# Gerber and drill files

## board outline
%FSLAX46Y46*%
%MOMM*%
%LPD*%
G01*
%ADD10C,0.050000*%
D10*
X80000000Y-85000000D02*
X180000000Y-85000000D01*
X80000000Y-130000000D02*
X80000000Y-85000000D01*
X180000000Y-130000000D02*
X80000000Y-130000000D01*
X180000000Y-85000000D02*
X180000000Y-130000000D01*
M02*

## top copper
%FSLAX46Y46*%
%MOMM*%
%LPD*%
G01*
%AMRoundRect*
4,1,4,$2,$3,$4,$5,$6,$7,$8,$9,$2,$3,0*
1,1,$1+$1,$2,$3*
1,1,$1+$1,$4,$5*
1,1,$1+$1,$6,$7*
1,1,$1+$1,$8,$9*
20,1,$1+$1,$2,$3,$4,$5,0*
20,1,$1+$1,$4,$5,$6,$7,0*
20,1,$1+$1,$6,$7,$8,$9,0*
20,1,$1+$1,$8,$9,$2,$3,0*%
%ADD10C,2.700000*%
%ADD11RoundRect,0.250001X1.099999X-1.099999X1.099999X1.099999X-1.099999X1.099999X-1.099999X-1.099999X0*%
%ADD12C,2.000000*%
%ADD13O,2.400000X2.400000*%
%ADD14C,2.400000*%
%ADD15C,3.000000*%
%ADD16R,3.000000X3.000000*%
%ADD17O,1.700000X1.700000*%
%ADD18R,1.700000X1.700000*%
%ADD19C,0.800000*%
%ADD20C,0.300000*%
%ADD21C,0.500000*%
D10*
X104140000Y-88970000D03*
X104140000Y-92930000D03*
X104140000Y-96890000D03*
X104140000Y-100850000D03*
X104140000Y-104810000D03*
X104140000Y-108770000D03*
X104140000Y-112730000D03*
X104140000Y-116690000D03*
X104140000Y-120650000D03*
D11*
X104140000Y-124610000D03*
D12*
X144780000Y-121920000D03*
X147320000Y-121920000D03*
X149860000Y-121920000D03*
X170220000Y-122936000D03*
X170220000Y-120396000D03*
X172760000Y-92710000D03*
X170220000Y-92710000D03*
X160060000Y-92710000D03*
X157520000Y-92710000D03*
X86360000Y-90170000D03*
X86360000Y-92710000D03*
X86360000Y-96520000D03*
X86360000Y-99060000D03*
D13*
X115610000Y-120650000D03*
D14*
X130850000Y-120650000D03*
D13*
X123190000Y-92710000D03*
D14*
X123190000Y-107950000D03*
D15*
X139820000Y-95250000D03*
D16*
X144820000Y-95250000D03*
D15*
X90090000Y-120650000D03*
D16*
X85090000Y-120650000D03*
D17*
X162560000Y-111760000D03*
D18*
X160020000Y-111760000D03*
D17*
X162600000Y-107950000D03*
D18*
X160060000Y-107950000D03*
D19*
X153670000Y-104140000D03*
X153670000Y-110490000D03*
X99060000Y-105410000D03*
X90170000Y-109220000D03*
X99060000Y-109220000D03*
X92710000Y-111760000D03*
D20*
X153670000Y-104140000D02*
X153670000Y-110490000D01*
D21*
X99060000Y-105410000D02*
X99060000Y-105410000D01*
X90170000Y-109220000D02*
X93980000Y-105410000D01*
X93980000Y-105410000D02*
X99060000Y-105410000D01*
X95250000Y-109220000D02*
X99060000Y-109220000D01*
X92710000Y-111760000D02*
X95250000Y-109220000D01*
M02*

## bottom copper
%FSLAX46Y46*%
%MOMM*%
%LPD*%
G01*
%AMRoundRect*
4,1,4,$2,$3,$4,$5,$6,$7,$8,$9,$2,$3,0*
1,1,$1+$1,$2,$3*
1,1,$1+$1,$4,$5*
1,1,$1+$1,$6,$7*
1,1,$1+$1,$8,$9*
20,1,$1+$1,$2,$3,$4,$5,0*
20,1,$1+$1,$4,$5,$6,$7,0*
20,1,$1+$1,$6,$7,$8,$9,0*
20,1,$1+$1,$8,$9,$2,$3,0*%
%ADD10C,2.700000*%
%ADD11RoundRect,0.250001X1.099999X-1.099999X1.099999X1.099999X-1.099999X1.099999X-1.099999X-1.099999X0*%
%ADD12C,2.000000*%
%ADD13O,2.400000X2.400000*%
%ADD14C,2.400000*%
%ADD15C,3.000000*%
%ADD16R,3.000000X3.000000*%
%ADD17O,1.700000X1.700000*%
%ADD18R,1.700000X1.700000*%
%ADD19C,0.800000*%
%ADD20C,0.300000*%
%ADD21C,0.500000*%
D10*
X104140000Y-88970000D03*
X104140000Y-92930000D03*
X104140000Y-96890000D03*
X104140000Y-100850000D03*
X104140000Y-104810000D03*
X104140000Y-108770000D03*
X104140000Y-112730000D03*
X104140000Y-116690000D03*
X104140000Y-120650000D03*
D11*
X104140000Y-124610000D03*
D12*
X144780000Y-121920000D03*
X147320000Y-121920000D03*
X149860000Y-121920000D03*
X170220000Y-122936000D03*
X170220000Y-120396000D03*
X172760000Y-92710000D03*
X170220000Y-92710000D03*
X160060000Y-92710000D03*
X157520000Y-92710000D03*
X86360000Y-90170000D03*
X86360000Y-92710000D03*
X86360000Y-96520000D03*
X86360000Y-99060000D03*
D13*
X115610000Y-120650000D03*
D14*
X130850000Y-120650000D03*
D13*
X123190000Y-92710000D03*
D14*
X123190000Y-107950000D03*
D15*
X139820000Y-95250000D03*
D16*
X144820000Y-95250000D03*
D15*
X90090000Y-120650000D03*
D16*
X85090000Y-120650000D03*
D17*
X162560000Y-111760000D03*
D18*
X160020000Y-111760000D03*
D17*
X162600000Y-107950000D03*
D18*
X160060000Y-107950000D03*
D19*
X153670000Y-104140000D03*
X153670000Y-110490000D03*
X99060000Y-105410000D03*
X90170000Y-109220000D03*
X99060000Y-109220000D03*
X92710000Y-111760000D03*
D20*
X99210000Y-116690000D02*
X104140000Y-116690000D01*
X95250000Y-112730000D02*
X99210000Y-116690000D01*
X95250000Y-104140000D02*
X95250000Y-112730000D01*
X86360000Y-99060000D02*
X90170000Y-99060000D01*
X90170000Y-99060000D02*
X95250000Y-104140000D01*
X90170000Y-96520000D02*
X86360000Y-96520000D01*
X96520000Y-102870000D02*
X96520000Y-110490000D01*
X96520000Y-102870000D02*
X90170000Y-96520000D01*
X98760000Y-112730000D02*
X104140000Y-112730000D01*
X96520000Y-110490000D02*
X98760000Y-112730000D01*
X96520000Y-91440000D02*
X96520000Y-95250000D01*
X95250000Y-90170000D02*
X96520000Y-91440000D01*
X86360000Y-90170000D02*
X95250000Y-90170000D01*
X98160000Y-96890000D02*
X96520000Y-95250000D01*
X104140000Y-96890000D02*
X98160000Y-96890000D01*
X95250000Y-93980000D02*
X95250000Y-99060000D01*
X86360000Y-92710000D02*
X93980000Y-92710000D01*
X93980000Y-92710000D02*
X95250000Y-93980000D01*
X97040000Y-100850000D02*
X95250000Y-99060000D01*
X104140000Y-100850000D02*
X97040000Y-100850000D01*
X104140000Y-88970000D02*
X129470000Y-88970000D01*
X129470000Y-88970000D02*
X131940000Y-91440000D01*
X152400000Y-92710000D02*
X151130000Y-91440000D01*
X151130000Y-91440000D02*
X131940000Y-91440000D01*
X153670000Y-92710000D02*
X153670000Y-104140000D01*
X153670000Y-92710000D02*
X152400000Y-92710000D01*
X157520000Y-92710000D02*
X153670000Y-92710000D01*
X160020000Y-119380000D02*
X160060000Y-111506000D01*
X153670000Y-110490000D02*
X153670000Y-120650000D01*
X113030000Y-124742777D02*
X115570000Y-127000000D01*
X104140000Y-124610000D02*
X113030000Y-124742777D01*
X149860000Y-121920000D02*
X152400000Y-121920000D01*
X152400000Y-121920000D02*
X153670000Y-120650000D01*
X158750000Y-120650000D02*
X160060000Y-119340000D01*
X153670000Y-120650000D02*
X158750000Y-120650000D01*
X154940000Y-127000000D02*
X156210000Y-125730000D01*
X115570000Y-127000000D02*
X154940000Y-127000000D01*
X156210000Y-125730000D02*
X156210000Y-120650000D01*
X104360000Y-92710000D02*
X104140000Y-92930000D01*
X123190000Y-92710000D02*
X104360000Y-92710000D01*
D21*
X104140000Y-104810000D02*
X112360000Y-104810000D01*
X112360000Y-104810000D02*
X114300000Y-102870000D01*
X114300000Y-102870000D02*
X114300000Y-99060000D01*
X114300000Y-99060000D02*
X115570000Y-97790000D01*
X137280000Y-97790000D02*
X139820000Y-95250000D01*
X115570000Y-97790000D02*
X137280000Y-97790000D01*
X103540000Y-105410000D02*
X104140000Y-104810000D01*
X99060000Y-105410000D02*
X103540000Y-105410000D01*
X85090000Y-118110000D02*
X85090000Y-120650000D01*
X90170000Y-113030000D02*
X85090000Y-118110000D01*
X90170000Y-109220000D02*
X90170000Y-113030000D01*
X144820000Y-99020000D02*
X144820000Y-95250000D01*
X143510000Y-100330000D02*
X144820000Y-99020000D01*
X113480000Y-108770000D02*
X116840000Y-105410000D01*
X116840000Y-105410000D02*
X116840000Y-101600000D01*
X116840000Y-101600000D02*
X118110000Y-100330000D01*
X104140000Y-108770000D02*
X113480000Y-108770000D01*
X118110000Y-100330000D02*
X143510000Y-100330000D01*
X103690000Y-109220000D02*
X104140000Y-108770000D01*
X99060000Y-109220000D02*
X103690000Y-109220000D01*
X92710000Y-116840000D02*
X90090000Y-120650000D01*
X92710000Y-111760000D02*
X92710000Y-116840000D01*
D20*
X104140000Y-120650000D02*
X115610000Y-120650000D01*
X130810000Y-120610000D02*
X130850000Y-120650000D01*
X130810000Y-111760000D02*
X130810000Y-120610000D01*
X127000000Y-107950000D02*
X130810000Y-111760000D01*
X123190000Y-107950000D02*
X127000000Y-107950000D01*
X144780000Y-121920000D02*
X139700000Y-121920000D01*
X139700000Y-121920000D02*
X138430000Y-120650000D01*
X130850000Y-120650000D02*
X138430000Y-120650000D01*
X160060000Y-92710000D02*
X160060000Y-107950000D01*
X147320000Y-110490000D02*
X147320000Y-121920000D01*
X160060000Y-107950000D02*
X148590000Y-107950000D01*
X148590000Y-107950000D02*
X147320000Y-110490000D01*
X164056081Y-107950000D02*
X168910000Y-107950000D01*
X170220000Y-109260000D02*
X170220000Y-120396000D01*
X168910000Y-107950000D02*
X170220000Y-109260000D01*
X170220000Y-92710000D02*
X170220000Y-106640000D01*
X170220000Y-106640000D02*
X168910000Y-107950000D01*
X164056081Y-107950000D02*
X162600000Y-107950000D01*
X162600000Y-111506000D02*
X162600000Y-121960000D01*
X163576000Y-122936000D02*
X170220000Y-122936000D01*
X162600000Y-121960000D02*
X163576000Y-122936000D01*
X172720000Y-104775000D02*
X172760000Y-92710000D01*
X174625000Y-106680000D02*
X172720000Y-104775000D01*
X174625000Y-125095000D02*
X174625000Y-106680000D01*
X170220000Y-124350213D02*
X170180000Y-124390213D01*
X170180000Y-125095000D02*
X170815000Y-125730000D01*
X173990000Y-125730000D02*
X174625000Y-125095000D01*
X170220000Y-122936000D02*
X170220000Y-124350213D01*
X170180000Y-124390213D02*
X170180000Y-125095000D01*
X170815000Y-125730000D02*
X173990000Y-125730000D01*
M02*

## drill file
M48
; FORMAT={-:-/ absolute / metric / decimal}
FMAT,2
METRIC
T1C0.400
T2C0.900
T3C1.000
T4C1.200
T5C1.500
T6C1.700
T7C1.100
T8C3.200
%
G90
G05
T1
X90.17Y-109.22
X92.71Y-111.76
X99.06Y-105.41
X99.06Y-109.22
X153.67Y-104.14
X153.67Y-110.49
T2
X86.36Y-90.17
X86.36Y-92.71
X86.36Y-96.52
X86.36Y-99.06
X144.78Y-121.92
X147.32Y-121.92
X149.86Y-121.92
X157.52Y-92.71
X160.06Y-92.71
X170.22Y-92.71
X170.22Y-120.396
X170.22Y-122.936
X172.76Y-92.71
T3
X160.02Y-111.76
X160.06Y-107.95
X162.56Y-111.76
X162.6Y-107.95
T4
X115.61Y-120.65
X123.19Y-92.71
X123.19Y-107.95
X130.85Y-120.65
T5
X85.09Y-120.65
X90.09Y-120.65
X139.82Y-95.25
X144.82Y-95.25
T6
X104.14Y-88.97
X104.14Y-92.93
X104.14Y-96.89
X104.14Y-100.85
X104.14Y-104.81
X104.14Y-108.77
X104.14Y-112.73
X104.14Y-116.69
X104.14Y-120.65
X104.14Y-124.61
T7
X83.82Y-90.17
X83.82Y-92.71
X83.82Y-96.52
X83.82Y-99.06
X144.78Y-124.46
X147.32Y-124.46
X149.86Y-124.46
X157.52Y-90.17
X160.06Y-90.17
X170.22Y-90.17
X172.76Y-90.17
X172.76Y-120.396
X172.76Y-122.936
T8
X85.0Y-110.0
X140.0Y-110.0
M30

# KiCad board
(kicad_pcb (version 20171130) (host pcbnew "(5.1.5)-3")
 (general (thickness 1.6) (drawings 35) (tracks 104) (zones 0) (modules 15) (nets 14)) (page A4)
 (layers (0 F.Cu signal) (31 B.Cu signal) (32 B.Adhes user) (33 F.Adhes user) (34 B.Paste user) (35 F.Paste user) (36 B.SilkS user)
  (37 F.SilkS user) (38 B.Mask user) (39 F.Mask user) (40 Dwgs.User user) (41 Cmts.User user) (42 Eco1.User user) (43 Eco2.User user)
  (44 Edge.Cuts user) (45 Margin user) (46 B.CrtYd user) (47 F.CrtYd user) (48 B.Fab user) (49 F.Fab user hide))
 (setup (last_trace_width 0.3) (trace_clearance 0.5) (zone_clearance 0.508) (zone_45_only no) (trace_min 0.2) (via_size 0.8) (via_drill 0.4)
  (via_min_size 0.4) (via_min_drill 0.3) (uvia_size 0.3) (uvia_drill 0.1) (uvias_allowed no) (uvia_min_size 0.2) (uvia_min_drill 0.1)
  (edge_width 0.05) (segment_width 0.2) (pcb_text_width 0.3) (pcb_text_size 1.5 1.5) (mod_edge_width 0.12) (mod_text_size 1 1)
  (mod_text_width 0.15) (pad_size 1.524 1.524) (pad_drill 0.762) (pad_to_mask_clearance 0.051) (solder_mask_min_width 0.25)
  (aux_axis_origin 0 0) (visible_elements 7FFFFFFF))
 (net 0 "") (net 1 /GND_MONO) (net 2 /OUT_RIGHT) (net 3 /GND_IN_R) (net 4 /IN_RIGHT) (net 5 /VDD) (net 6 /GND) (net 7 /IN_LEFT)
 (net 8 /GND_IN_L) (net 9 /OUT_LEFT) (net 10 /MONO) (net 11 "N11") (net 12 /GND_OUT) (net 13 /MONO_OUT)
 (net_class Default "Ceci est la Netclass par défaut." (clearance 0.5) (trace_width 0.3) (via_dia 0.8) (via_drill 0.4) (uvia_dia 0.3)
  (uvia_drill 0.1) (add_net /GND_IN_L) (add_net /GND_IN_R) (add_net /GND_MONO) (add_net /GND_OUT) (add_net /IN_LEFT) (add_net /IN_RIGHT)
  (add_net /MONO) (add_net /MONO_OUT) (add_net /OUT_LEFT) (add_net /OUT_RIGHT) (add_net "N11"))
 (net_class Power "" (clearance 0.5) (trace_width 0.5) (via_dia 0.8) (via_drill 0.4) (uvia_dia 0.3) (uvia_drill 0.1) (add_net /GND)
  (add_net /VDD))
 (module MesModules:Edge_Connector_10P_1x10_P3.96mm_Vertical (layer F.Cu) (at 104.14 124.61 90)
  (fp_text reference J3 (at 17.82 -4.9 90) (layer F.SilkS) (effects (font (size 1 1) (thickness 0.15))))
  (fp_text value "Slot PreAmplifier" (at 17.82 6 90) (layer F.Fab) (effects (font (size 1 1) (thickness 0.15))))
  (pad 10 thru_hole circle (at 35.64 0 90) (size 2.7 2.7) (drill 1.7) (layers *.Cu *.Mask) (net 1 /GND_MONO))
  (pad 9 thru_hole circle (at 31.68 0 90) (size 2.7 2.7) (drill 1.7) (layers *.Cu *.Mask) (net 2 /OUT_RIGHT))
  (pad 8 thru_hole circle (at 27.72 0 90) (size 2.7 2.7) (drill 1.7) (layers *.Cu *.Mask) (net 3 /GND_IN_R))
  (pad 7 thru_hole circle (at 23.76 0 90) (size 2.7 2.7) (drill 1.7) (layers *.Cu *.Mask) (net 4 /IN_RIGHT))
  (pad 6 thru_hole circle (at 19.8 0 90) (size 2.7 2.7) (drill 1.7) (layers *.Cu *.Mask) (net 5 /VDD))
  (pad 5 thru_hole circle (at 15.84 0 90) (size 2.7 2.7) (drill 1.7) (layers *.Cu *.Mask) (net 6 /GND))
  (pad 4 thru_hole circle (at 11.88 0 90) (size 2.7 2.7) (drill 1.7) (layers *.Cu *.Mask) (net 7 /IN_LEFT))
  (pad 3 thru_hole circle (at 7.92 0 90) (size 2.7 2.7) (drill 1.7) (layers *.Cu *.Mask) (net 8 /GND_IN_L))
  (pad 2 thru_hole circle (at 3.96 0 90) (size 2.7 2.7) (drill 1.7) (layers *.Cu *.Mask) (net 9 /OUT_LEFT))
  (pad 1 thru_hole roundrect (at 0 0 90) (size 2.7 2.7) (drill 1.7) (layers *.Cu *.Mask) (roundrect_rratio 0.09259299999999999)
   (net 1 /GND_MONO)))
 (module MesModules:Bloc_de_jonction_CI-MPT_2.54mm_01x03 (layer F.Cu) (at 149.86 121.92 180)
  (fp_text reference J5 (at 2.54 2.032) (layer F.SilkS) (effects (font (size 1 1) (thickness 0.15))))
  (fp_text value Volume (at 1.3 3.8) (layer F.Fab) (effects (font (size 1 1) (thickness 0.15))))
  (pad "" np_thru_hole circle (at 5.08 -2.54 180) (size 1.1 1.1) (drill 1.1) (layers *.Cu *.Mask))
  (pad 3 thru_hole circle (at 5.08 0 180) (size 2 2) (drill 0.9) (layers *.Cu *.Mask) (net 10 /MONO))
  (pad "" np_thru_hole circle (at 2.54 -2.54 180) (size 1.1 1.1) (drill 1.1) (layers *.Cu *.Mask))
  (pad "" np_thru_hole circle (at 0 -2.54 180) (size 1.1 1.1) (drill 1.1) (layers *.Cu *.Mask))
  (pad 2 thru_hole circle (at 2.54 0 180) (size 2 2) (drill 0.9) (layers *.Cu *.Mask) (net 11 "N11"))
  (pad 1 thru_hole circle (at 0 0 180) (size 2 2) (drill 0.9) (layers *.Cu *.Mask) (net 1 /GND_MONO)))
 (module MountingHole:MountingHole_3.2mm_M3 (layer F.Cu) (at 140 110)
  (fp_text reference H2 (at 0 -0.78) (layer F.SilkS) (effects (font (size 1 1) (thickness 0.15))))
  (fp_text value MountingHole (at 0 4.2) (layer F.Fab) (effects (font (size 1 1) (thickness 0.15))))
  (pad 1 np_thru_hole circle (at 0 0) (size 3.2 3.2) (drill 3.2) (layers *.Cu *.Mask)))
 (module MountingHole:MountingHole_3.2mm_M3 (layer F.Cu) (at 85 110)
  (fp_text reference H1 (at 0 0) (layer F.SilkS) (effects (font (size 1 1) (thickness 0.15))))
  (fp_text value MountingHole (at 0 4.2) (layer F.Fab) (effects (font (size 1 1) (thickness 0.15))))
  (pad 1 np_thru_hole circle (at 0 0) (size 3.2 3.2) (drill 3.2) (layers *.Cu *.Mask)))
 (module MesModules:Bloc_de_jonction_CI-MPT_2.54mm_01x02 (layer F.Cu) (at 170.22 120.396 270)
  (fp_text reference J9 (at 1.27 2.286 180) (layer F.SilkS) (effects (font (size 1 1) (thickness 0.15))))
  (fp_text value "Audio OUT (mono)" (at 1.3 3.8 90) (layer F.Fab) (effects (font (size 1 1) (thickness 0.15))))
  (pad "" np_thru_hole circle (at 2.54 -2.54 270) (size 1.1 1.1) (drill 1.1) (layers *.Cu *.Mask))
  (pad "" np_thru_hole circle (at 0 -2.54 270) (size 1.1 1.1) (drill 1.1) (layers *.Cu *.Mask))
  (pad 2 thru_hole circle (at 2.54 0 270) (size 2 2) (drill 0.9) (layers *.Cu *.Mask) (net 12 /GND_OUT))
  (pad 1 thru_hole circle (at 0 0 270) (size 2 2) (drill 0.9) (layers *.Cu *.Mask) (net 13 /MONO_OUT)))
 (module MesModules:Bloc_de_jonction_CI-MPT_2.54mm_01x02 (layer F.Cu) (at 170.22 92.71)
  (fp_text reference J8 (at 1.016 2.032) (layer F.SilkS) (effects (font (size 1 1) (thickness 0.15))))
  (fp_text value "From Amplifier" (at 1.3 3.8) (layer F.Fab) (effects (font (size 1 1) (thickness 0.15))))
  (pad "" np_thru_hole circle (at 2.54 -2.54) (size 1.1 1.1) (drill 1.1) (layers *.Cu *.Mask))
  (pad "" np_thru_hole circle (at 0 -2.54) (size 1.1 1.1) (drill 1.1) (layers *.Cu *.Mask))
  (pad 2 thru_hole circle (at 2.54 0) (size 2 2) (drill 0.9) (layers *.Cu *.Mask) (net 12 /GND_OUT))
  (pad 1 thru_hole circle (at 0 0) (size 2 2) (drill 0.9) (layers *.Cu *.Mask) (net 13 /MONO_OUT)))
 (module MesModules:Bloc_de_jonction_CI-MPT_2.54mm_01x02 (layer F.Cu) (at 157.52 92.71)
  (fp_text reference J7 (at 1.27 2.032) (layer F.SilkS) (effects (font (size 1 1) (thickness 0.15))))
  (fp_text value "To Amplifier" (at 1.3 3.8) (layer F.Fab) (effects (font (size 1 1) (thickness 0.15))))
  (pad "" np_thru_hole circle (at 2.54 -2.54) (size 1.1 1.1) (drill 1.1) (layers *.Cu *.Mask))
  (pad "" np_thru_hole circle (at 0 -2.54) (size 1.1 1.1) (drill 1.1) (layers *.Cu *.Mask))
  (pad 2 thru_hole circle (at 2.54 0) (size 2 2) (drill 0.9) (layers *.Cu *.Mask) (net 11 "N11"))
  (pad 1 thru_hole circle (at 0 0) (size 2 2) (drill 0.9) (layers *.Cu *.Mask) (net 1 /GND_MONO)))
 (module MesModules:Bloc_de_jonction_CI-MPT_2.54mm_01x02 (layer F.Cu) (at 86.36 92.71 90)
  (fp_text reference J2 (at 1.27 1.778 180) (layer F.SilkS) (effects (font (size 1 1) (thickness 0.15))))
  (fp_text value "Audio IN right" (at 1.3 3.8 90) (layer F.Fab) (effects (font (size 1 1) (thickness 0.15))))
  (pad "" np_thru_hole circle (at 2.54 -2.54 90) (size 1.1 1.1) (drill 1.1) (layers *.Cu *.Mask))
  (pad "" np_thru_hole circle (at 0 -2.54 90) (size 1.1 1.1) (drill 1.1) (layers *.Cu *.Mask))
  (pad 2 thru_hole circle (at 2.54 0 90) (size 2 2) (drill 0.9) (layers *.Cu *.Mask) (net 3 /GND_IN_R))
  (pad 1 thru_hole circle (at 0 0 90) (size 2 2) (drill 0.9) (layers *.Cu *.Mask) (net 4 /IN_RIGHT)))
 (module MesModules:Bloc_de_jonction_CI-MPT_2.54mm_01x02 (layer F.Cu) (at 86.36 99.06 90)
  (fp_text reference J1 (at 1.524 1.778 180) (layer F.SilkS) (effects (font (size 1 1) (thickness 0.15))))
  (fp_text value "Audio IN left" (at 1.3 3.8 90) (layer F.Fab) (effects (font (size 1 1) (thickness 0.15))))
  (pad "" np_thru_hole circle (at 2.54 -2.54 90) (size 1.1 1.1) (drill 1.1) (layers *.Cu *.Mask))
  (pad "" np_thru_hole circle (at 0 -2.54 90) (size 1.1 1.1) (drill 1.1) (layers *.Cu *.Mask))
  (pad 2 thru_hole circle (at 2.54 0 90) (size 2 2) (drill 0.9) (layers *.Cu *.Mask) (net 7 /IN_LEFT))
  (pad 1 thru_hole circle (at 0 0 90) (size 2 2) (drill 0.9) (layers *.Cu *.Mask) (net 8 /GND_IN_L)))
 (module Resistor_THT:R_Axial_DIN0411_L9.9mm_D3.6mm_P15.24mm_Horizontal (layer F.Cu) (at 130.85 120.65 180)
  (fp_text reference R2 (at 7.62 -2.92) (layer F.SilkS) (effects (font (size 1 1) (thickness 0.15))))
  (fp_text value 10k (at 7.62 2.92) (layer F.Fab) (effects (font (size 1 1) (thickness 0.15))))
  (pad 2 thru_hole oval (at 15.24 0 180) (size 2.4 2.4) (drill 1.2) (layers *.Cu *.Mask) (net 9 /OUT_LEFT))
  (pad 1 thru_hole circle (at 0 0 180) (size 2.4 2.4) (drill 1.2) (layers *.Cu *.Mask) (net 10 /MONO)))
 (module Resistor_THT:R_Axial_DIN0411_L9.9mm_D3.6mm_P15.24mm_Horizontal (layer F.Cu) (at 123.19 107.95 90)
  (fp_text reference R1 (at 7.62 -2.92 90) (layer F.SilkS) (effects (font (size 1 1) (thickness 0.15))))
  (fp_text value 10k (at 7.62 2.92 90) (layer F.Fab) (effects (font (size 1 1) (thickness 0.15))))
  (pad 2 thru_hole oval (at 15.24 0 90) (size 2.4 2.4) (drill 1.2) (layers *.Cu *.Mask) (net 2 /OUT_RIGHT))
  (pad 1 thru_hole circle (at 0 0 90) (size 2.4 2.4) (drill 1.2) (layers *.Cu *.Mask) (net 10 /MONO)))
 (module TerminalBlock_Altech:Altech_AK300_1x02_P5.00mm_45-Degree (layer F.Cu) (at 144.82 95.25 180)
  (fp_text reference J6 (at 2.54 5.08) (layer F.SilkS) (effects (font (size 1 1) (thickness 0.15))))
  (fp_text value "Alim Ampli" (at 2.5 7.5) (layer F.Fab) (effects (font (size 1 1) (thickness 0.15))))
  (pad 2 thru_hole circle (at 5 0 180) (size 3 3) (drill 1.5) (layers *.Cu *.Mask) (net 5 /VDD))
  (pad 1 thru_hole rect (at 0 0 180) (size 3 3) (drill 1.5) (layers *.Cu *.Mask) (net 6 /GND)))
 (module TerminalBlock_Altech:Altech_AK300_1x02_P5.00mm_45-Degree (layer F.Cu) (at 85.09 120.65)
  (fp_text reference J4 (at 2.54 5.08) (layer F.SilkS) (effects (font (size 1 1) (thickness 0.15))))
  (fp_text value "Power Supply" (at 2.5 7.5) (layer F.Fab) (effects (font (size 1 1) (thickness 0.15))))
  (pad 2 thru_hole circle (at 5 0) (size 3 3) (drill 1.5) (layers *.Cu *.Mask) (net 6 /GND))
  (pad 1 thru_hole rect (at 0 0) (size 3 3) (drill 1.5) (layers *.Cu *.Mask) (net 5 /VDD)))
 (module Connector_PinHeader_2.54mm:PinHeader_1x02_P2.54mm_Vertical (layer F.Cu) (at 160.02 111.76 90)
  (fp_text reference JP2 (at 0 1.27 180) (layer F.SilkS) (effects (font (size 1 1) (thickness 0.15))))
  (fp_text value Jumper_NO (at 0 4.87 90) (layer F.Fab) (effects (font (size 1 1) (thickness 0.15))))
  (pad 2 thru_hole oval (at 0 2.54 90) (size 1.7 1.7) (drill 1) (layers *.Cu *.Mask) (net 12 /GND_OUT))
  (pad 1 thru_hole rect (at 0 0 90) (size 1.7 1.7) (drill 1) (layers *.Cu *.Mask) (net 1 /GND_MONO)))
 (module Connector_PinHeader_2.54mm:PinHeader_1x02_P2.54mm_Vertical (layer F.Cu) (at 160.06 107.95 90)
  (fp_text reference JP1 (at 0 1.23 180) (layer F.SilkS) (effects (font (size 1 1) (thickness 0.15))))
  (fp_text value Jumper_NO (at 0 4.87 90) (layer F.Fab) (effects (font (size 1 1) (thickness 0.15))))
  (pad 2 thru_hole oval (at 0 2.54 90) (size 1.7 1.7) (drill 1) (layers *.Cu *.Mask) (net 13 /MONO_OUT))
  (pad 1 thru_hole rect (at 0 0 90) (size 1.7 1.7) (drill 1) (layers *.Cu *.Mask) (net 11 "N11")))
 (gr_line (start 80 85) (end 180 85) (layer Edge.Cuts) (width 0.05))
 (gr_line (start 80 130) (end 80 85) (layer Edge.Cuts) (width 0.05))
 (gr_line (start 180 130) (end 80 130) (layer Edge.Cuts) (width 0.05))
 (gr_line (start 180 85) (end 180 130) (layer Edge.Cuts) (width 0.05))
 (segment (start 99.21 116.69) (end 104.14 116.69) (width 0.3) (layer B.Cu) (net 8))
 (segment (start 95.25 112.73) (end 99.21 116.69) (width 0.3) (layer B.Cu) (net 8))
 (segment (start 95.25 104.14) (end 95.25 112.73) (width 0.3) (layer B.Cu) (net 8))
 (segment (start 86.36 99.06) (end 90.17 99.06) (width 0.3) (layer B.Cu) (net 8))
 (segment (start 90.17 99.06) (end 95.25 104.14) (width 0.3) (layer B.Cu) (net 8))
 (segment (start 90.17 96.52) (end 86.36 96.52) (width 0.3) (layer B.Cu) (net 7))
 (segment (start 96.52 102.87) (end 96.52 110.49) (width 0.3) (layer B.Cu) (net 7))
 (segment (start 96.52 102.87) (end 90.17 96.52) (width 0.3) (layer B.Cu) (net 7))
 (segment (start 98.76 112.73) (end 104.14 112.73) (width 0.3) (layer B.Cu) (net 7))
 (segment (start 96.52 110.49) (end 98.76 112.73) (width 0.3) (layer B.Cu) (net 7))
 (segment (start 96.52 91.44) (end 96.52 95.25) (width 0.3) (layer B.Cu) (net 3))
 (segment (start 95.25 90.17) (end 96.52 91.44) (width 0.3) (layer B.Cu) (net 3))
 (segment (start 86.36 90.17) (end 95.25 90.17) (width 0.3) (layer B.Cu) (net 3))
 (segment (start 98.16 96.89) (end 96.52 95.25) (width 0.3) (layer B.Cu) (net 3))
 (segment (start 104.14 96.89) (end 98.16 96.89) (width 0.3) (layer B.Cu) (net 3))
 (segment (start 95.25 93.98) (end 95.25 99.06) (width 0.3) (layer B.Cu) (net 4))
 (segment (start 86.36 92.71) (end 93.98 92.71) (width 0.3) (layer B.Cu) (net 4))
 (segment (start 93.98 92.71) (end 95.25 93.98) (width 0.3) (layer B.Cu) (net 4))
 (segment (start 97.04 100.85) (end 95.25 99.06) (width 0.3) (layer B.Cu) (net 4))
 (segment (start 104.14 100.85) (end 97.04 100.85) (width 0.3) (layer B.Cu) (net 4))
 (segment (start 104.14 88.97) (end 129.47 88.97) (width 0.3) (layer B.Cu) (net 1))
 (segment (start 129.47 88.97) (end 131.94 91.44) (width 0.3) (layer B.Cu) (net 1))
 (segment (start 152.4 92.71) (end 151.13 91.44) (width 0.3) (layer B.Cu) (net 1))
 (segment (start 151.13 91.44) (end 131.94 91.44) (width 0.3) (layer B.Cu) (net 1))
 (via (at 153.67 104.14) (size 0.8) (drill 0.4) (layers F.Cu B.Cu) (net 1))
 (segment (start 153.67 92.71) (end 153.67 104.14) (width 0.3) (layer B.Cu) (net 1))
 (segment (start 153.67 92.71) (end 152.4 92.71) (width 0.3) (layer B.Cu) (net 1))
 (segment (start 157.52 92.71) (end 153.67 92.71) (width 0.3) (layer B.Cu) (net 1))
 (via (at 153.67 110.49) (size 0.8) (drill 0.4) (layers F.Cu B.Cu) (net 1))
 (segment (start 153.67 104.14) (end 153.67 110.49) (width 0.3) (layer F.Cu) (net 1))
 (segment (start 160.02 119.38) (end 160.06 111.506) (width 0.3) (layer B.Cu) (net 1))
 (segment (start 153.67 110.49) (end 153.67 120.65) (width 0.3) (layer B.Cu) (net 1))
 (segment (start 113.03 124.742777) (end 115.57 127) (width 0.3) (layer B.Cu) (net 1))
 (segment (start 104.14 124.61) (end 113.03 124.742777) (width 0.3) (layer B.Cu) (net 1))
 (segment (start 149.86 121.92) (end 152.4 121.92) (width 0.3) (layer B.Cu) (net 1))
 (segment (start 152.4 121.92) (end 153.67 120.65) (width 0.3) (layer B.Cu) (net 1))
 (segment (start 158.75 120.65) (end 160.06 119.34) (width 0.3) (layer B.Cu) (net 1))
 (segment (start 153.67 120.65) (end 158.75 120.65) (width 0.3) (layer B.Cu) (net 1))
 (segment (start 154.94 127) (end 156.21 125.73) (width 0.3) (layer B.Cu) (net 1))
 (segment (start 115.57 127) (end 154.94 127) (width 0.3) (layer B.Cu) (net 1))
 (segment (start 156.21 125.73) (end 156.21 120.65) (width 0.3) (layer B.Cu) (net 1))
 (segment (start 104.36 92.71) (end 104.14 92.93) (width 0.3) (layer B.Cu) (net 2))
 (segment (start 123.19 92.71) (end 104.36 92.71) (width 0.3) (layer B.Cu) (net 2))
 (segment (start 104.14 104.81) (end 112.36 104.81) (width 0.5) (layer B.Cu) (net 5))
 (segment (start 112.36 104.81) (end 114.3 102.87) (width 0.5) (layer B.Cu) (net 5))
 (segment (start 114.3 102.87) (end 114.3 99.06) (width 0.5) (layer B.Cu) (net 5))
 (segment (start 114.3 99.06) (end 115.57 97.79) (width 0.5) (layer B.Cu) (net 5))
 (segment (start 137.28 97.79) (end 139.82 95.25) (width 0.5) (layer B.Cu) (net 5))
 (segment (start 115.57 97.79) (end 137.28 97.79) (width 0.5) (layer B.Cu) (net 5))
 (segment (start 99.06 105.41) (end 99.06 105.41) (width 0.5) (layer F.Cu) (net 5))
 (via (at 99.06 105.41) (size 0.8) (drill 0.4) (layers F.Cu B.Cu) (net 5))
 (segment (start 103.54 105.41) (end 104.14 104.81) (width 0.5) (layer B.Cu) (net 5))
 (segment (start 99.06 105.41) (end 103.54 105.41) (width 0.5) (layer B.Cu) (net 5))
 (segment (start 90.17 109.22) (end 93.98 105.41) (width 0.5) (layer F.Cu) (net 5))
 (via (at 90.17 109.22) (size 0.8) (drill 0.4) (layers F.Cu B.Cu) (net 5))
 (segment (start 93.98 105.41) (end 99.06 105.41) (width 0.5) (layer F.Cu) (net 5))
 (segment (start 85.09 118.11) (end 85.09 120.65) (width 0.5) (layer B.Cu) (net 5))
 (segment (start 90.17 113.03) (end 85.09 118.11) (width 0.5) (layer B.Cu) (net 5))
 (segment (start 90.17 109.22) (end 90.17 113.03) (width 0.5) (layer B.Cu) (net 5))
 (segment (start 144.82 99.02) (end 144.82 95.25) (width 0.5) (layer B.Cu) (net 6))
 (segment (start 143.51 100.33) (end 144.82 99.02) (width 0.5) (layer B.Cu) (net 6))
 (segment (start 113.48 108.77) (end 116.84 105.41) (width 0.5) (layer B.Cu) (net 6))
 (segment (start 116.84 105.41) (end 116.84 101.6) (width 0.5) (layer B.Cu) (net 6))
 (segment (start 116.84 101.6) (end 118.11 100.33) (width 0.5) (layer B.Cu) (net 6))
 (segment (start 104.14 108.77) (end 113.48 108.77) (width 0.5) (layer B.Cu) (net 6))
 (segment (start 118.11 100.33) (end 143.51 100.33) (width 0.5) (layer B.Cu) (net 6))
 (segment (start 103.69 109.22) (end 104.14 108.77) (width 0.5) (layer B.Cu) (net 6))
 (segment (start 99.06 109.22) (end 103.69 109.22) (width 0.5) (layer B.Cu) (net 6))
 (via (at 99.06 109.22) (size 0.8) (drill 0.4) (layers F.Cu B.Cu) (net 6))
 (via (at 92.71 111.76) (size 0.8) (drill 0.4) (layers F.Cu B.Cu) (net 6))
 (segment (start 95.25 109.22) (end 99.06 109.22) (width 0.5) (layer F.Cu) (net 6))
 (segment (start 92.71 111.76) (end 95.25 109.22) (width 0.5) (layer F.Cu) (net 6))
 (segment (start 92.71 116.84) (end 90.09 120.65) (width 0.5) (layer B.Cu) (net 6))
 (segment (start 92.71 111.76) (end 92.71 116.84) (width 0.5) (layer B.Cu) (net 6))
 (segment (start 104.14 120.65) (end 115.61 120.65) (width 0.3) (layer B.Cu) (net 9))
 (segment (start 130.81 120.61) (end 130.85 120.65) (width 0.3) (layer B.Cu) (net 10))
 (segment (start 130.81 111.76) (end 130.81 120.61) (width 0.3) (layer B.Cu) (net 10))
 (segment (start 127 107.95) (end 130.81 111.76) (width 0.3) (layer B.Cu) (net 10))
 (segment (start 123.19 107.95) (end 127 107.95) (width 0.3) (layer B.Cu) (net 10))
 (segment (start 144.78 121.92) (end 139.7 121.92) (width 0.3) (layer B.Cu) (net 10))
 (segment (start 139.7 121.92) (end 138.43 120.65) (width 0.3) (layer B.Cu) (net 10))
 (segment (start 130.85 120.65) (end 138.43 120.65) (width 0.3) (layer B.Cu) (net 10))
 (segment (start 160.06 92.71) (end 160.06 107.95) (width 0.3) (layer B.Cu) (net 11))
 (segment (start 147.32 110.49) (end 147.32 121.92) (width 0.3) (layer B.Cu) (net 11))
 (segment (start 160.06 107.95) (end 148.59 107.95) (width 0.3) (layer B.Cu) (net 11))
 (segment (start 148.59 107.95) (end 147.32 110.49) (width 0.3) (layer B.Cu) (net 11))
 (segment (start 164.056081 107.95) (end 168.91 107.95) (width 0.3) (layer B.Cu) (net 13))
 (segment (start 170.22 109.26) (end 170.22 120.396) (width 0.3) (layer B.Cu) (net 13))
 (segment (start 168.91 107.95) (end 170.22 109.26) (width 0.3) (layer B.Cu) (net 13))
 (segment (start 170.22 92.71) (end 170.22 106.64) (width 0.3) (layer B.Cu) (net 13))
 (segment (start 170.22 106.64) (end 168.91 107.95) (width 0.3) (layer B.Cu) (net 13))
 (segment (start 164.056081 107.95) (end 162.6 107.95) (width 0.3) (layer B.Cu) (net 13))
 (segment (start 162.6 111.506) (end 162.6 121.96) (width 0.3) (layer B.Cu) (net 12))
 (segment (start 163.576 122.936) (end 170.22 122.936) (width 0.3) (layer B.Cu) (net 12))
 (segment (start 162.6 121.96) (end 163.576 122.936) (width 0.3) (layer B.Cu) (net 12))
 (segment (start 172.72 104.775) (end 172.76 92.71) (width 0.3) (layer B.Cu) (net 12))
 (segment (start 174.625 106.68) (end 172.72 104.775) (width 0.3) (layer B.Cu) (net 12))
 (segment (start 174.625 125.095) (end 174.625 106.68) (width 0.3) (layer B.Cu) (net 12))
 (segment (start 170.22 124.350213) (end 170.18 124.390213) (width 0.3) (layer B.Cu) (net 12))
 (segment (start 170.18 125.095) (end 170.815 125.73) (width 0.3) (layer B.Cu) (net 12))
 (segment (start 173.99 125.73) (end 174.625 125.095) (width 0.3) (layer B.Cu) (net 12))
 (segment (start 170.22 122.936) (end 170.22 124.350213) (width 0.3) (layer B.Cu) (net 12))
 (segment (start 170.18 124.390213) (end 170.18 125.095) (width 0.3) (layer B.Cu) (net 12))
 (segment (start 170.815 125.73) (end 173.99 125.73) (width 0.3) (layer B.Cu) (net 12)))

